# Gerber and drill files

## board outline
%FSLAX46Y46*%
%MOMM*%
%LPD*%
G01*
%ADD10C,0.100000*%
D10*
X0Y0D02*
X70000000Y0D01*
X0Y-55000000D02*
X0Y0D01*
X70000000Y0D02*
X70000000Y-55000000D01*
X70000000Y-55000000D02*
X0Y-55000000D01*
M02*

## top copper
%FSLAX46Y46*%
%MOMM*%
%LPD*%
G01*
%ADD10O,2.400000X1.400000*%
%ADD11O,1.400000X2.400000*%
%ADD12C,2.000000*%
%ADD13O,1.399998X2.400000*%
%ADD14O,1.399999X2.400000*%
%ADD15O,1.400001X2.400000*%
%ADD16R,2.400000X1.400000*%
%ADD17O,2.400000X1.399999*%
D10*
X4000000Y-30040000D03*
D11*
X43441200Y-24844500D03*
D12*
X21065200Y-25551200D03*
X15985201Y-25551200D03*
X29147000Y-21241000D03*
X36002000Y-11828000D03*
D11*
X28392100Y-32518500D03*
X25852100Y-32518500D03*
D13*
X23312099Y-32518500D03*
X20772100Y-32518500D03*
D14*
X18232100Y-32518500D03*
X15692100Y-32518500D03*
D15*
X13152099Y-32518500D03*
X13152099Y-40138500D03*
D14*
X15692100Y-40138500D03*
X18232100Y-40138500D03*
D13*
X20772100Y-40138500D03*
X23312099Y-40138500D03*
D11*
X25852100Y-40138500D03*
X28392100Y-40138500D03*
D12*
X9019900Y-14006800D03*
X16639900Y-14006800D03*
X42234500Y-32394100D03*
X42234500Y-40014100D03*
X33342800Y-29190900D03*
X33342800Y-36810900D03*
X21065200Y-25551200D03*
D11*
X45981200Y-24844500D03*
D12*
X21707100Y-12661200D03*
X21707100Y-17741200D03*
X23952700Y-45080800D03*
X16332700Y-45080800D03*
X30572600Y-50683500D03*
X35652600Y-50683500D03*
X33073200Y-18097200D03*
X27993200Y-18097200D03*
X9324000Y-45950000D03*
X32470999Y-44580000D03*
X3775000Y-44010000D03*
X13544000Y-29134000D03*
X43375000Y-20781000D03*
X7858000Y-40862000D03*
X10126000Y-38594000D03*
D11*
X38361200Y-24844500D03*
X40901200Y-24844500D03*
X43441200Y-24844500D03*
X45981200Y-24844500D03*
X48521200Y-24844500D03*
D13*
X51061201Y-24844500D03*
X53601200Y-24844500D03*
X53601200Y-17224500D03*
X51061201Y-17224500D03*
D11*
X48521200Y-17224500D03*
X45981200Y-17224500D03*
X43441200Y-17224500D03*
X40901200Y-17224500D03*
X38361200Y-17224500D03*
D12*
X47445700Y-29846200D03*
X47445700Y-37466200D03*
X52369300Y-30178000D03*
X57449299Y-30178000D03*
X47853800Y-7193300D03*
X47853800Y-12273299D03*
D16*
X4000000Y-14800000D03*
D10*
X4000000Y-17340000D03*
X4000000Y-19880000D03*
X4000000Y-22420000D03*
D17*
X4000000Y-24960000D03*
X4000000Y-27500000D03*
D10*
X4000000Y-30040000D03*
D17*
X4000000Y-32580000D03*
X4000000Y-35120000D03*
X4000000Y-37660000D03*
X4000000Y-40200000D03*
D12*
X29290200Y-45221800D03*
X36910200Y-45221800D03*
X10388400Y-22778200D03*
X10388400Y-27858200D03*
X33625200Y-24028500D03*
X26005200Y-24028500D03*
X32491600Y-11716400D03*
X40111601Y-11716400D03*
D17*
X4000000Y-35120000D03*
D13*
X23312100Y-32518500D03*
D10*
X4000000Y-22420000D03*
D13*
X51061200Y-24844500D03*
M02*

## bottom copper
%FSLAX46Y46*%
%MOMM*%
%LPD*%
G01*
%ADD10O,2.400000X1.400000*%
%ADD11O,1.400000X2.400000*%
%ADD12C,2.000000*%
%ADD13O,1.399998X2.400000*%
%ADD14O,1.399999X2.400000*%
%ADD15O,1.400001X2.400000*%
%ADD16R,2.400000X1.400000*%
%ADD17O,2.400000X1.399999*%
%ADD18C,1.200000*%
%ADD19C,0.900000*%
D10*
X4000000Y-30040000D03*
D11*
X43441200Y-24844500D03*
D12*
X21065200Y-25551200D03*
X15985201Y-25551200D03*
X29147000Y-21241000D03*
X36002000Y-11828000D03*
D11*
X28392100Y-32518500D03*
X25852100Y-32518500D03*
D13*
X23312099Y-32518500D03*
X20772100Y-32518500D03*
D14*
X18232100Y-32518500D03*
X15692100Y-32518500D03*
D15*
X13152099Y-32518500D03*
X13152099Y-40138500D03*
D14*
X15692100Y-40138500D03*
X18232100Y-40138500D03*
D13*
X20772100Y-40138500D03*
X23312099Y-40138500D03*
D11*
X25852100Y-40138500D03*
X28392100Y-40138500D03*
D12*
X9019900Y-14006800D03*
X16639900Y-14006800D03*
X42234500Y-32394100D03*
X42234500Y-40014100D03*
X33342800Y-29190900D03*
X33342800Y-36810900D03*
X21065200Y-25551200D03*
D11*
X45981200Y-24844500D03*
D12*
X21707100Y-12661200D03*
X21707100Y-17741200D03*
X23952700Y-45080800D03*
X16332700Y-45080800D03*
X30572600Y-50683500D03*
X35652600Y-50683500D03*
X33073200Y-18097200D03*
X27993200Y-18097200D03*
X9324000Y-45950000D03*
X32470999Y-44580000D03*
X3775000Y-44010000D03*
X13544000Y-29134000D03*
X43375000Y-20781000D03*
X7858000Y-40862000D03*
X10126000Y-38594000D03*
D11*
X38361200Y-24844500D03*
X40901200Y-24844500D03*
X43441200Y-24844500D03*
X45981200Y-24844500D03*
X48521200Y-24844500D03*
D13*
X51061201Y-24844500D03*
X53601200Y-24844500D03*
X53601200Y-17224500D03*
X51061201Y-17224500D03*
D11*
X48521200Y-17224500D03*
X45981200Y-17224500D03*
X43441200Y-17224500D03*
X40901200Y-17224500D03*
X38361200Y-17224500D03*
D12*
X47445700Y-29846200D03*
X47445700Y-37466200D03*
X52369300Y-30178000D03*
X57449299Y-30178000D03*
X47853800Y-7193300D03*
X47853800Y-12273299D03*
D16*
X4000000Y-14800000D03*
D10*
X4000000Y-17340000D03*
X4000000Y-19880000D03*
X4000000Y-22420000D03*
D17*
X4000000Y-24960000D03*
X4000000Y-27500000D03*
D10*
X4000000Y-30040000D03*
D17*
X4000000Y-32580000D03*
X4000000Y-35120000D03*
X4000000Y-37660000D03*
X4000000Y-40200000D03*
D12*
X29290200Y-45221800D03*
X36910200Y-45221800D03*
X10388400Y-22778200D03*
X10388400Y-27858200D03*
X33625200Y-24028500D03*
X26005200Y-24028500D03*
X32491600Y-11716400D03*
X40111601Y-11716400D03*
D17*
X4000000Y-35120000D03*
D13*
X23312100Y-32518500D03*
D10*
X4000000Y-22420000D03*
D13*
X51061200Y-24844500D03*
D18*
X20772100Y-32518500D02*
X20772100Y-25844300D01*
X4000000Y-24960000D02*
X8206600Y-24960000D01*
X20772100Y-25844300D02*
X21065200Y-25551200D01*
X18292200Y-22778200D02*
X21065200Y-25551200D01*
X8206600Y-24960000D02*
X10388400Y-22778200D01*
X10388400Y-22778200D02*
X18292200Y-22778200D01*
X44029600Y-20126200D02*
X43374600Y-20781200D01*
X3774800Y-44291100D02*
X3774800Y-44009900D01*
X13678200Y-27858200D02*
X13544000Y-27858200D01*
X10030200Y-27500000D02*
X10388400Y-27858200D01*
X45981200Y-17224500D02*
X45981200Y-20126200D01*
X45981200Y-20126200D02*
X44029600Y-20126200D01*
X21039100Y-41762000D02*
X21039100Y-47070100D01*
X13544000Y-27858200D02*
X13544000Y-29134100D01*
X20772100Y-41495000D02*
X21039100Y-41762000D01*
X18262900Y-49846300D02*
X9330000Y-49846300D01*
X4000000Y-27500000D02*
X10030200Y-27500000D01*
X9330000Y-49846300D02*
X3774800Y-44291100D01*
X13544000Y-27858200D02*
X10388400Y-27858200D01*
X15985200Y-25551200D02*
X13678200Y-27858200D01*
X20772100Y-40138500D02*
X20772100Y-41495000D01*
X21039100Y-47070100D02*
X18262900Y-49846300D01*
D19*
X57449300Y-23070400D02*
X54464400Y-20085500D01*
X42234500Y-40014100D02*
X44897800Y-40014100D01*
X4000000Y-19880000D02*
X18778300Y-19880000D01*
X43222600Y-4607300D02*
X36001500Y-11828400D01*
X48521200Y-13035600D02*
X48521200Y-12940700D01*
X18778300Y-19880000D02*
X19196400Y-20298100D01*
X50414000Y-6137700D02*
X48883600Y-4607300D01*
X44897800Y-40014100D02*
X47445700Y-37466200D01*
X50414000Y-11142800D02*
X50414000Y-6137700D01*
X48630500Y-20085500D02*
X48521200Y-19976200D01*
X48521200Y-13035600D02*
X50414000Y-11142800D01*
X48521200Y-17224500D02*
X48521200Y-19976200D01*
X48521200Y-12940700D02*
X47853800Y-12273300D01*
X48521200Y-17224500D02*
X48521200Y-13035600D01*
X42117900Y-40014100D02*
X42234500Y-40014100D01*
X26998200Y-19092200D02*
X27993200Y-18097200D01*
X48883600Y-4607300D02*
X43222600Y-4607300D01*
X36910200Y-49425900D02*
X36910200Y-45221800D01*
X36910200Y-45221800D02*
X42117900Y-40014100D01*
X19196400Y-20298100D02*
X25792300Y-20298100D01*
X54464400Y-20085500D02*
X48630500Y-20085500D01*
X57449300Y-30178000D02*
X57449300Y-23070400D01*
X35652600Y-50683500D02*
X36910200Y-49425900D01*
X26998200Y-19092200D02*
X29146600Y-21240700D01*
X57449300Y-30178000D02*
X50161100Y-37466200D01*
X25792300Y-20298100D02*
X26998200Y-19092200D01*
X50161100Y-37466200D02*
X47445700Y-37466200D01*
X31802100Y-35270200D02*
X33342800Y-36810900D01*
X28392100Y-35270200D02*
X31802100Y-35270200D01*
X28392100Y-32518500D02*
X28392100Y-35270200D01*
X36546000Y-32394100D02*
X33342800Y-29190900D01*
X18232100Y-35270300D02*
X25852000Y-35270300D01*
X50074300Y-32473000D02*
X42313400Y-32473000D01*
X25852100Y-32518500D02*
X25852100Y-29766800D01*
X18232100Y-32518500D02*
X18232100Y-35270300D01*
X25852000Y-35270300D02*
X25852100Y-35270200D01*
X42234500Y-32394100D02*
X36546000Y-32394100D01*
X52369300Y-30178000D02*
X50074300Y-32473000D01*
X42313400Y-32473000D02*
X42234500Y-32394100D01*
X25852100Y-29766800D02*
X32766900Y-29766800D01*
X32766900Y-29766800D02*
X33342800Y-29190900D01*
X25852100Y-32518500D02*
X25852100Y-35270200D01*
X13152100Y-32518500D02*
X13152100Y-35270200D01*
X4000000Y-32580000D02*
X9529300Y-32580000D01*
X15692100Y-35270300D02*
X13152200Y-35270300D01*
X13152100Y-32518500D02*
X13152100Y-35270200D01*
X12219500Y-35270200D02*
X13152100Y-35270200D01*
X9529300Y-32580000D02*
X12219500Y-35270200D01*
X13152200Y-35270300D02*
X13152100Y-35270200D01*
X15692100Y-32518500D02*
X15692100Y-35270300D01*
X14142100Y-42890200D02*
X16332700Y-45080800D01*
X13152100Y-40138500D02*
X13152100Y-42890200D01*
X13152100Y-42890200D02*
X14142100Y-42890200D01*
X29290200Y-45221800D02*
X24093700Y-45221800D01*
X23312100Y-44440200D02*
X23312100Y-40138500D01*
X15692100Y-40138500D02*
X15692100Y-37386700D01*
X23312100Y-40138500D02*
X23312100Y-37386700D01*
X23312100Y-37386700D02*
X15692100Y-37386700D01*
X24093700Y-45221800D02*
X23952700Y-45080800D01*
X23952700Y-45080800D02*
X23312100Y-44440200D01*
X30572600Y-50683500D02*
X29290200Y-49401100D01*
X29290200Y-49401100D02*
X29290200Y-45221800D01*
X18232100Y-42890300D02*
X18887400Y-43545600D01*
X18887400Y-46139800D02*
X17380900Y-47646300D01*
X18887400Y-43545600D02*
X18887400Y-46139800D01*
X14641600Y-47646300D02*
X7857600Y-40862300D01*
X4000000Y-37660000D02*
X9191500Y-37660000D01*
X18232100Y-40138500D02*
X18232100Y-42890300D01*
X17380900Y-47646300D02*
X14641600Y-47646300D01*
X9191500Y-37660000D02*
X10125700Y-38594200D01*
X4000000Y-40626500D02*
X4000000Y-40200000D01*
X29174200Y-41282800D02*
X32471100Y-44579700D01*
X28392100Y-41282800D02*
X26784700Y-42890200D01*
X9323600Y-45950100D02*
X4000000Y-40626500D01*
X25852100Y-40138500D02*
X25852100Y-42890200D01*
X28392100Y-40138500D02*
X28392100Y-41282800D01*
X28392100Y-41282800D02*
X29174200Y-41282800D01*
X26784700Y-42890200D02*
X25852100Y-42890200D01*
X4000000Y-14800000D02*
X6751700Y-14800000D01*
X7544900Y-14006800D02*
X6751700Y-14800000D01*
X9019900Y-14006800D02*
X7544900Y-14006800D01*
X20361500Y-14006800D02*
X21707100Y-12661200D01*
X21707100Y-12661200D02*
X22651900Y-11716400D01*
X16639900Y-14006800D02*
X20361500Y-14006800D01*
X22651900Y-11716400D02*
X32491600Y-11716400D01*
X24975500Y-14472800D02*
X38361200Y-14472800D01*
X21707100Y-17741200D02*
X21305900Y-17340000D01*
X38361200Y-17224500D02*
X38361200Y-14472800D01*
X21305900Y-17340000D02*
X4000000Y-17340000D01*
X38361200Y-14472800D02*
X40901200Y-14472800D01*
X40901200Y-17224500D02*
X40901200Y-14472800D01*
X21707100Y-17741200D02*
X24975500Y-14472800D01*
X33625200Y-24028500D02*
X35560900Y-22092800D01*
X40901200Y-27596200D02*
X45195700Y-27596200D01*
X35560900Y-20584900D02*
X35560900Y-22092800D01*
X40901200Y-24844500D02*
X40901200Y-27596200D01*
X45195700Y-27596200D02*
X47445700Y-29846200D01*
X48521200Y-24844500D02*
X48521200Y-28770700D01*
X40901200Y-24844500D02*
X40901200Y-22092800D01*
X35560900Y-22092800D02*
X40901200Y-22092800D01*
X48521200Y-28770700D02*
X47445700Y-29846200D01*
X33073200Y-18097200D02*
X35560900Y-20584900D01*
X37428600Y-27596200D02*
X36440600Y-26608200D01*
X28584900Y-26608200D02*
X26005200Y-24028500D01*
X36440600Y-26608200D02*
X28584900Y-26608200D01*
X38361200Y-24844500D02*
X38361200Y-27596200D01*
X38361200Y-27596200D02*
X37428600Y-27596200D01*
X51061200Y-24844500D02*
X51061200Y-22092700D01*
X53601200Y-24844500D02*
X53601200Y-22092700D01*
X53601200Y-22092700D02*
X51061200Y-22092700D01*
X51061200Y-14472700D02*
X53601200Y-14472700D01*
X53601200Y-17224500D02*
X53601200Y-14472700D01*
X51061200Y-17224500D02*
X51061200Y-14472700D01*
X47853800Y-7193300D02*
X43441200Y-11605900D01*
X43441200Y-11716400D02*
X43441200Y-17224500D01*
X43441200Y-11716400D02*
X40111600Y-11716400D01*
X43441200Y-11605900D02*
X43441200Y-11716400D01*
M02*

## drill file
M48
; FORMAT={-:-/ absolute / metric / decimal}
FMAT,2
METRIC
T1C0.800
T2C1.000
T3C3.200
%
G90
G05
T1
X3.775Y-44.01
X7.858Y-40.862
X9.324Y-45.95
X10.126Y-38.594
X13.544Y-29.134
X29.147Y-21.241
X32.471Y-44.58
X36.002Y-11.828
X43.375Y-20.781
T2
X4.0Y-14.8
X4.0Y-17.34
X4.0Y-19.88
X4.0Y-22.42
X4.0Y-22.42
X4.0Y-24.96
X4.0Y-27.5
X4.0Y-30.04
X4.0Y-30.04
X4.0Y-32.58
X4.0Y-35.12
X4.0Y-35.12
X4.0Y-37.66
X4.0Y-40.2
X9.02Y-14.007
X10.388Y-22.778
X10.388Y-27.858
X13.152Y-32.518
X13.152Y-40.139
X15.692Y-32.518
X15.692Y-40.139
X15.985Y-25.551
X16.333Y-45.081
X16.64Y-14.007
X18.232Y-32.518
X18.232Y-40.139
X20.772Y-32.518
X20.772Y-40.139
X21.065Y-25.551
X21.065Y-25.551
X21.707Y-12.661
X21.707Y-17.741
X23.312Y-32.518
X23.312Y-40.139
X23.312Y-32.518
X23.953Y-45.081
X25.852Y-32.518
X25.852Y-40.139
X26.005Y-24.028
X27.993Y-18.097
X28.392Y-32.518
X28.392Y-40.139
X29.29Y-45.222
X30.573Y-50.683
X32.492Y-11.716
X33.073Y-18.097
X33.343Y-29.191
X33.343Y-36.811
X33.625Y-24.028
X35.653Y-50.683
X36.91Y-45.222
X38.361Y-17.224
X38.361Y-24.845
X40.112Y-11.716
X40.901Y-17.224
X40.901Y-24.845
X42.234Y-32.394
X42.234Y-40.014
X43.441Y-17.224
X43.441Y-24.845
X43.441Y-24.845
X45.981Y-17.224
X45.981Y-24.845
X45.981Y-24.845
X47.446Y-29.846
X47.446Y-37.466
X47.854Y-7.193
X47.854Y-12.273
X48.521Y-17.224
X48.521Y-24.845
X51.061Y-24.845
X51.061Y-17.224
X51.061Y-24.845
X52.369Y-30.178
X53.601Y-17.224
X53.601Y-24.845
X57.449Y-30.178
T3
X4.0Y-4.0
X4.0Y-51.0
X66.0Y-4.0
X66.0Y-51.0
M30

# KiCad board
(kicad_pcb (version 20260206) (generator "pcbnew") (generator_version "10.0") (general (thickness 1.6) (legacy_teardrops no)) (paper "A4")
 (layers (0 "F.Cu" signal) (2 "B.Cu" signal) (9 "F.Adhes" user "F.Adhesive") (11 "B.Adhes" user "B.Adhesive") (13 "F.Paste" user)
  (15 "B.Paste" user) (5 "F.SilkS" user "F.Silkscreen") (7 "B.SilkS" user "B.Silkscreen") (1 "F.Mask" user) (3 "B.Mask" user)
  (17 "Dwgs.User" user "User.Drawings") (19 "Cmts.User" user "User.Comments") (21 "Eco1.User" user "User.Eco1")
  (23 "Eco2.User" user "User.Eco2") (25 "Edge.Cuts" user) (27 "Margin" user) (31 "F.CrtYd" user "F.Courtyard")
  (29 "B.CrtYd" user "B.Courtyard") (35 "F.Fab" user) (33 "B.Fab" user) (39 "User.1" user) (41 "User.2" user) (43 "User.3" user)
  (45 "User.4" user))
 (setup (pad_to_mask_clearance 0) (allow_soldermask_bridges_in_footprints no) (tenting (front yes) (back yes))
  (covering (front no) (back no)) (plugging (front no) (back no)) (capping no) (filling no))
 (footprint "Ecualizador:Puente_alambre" (layer "F.Cu") (at 4 30.04)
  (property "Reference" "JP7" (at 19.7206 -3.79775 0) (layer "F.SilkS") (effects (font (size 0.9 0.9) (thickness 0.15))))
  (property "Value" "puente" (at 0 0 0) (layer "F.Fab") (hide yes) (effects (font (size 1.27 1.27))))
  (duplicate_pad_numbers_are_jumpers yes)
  (pad "1" thru_hole oval (at 0 0) (size 2.4 1.4) (drill 1) (layers "*.Cu" "*.Mask") (remove_unused_layers no) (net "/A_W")
   (thermal_bridge_angle 45))
  (pad "1" thru_hole oval (at 39.4412 -5.1955 90) (size 2.4 1.4) (drill 1) (layers "*.Cu" "*.Mask") (remove_unused_layers no) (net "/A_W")
   (thermal_bridge_angle 45)))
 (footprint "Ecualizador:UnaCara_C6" (layer "F.Cu") (at 21.0652 25.5512 180)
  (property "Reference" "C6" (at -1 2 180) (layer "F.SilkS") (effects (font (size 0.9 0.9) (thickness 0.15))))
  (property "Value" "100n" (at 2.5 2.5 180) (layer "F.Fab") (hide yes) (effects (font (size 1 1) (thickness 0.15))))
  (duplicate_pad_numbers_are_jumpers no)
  (pad "1" thru_hole circle (at 0 0 180) (size 2 2) (drill 1) (layers "*.Cu" "*.Mask") (remove_unused_layers no) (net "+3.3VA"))
  (pad "2" thru_hole circle (at 5.079999 0 180) (size 2 2) (drill 1) (layers "*.Cu" "*.Mask") (remove_unused_layers no) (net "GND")))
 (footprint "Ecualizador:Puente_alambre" (layer "F.Cu") (at 29.147 21.241)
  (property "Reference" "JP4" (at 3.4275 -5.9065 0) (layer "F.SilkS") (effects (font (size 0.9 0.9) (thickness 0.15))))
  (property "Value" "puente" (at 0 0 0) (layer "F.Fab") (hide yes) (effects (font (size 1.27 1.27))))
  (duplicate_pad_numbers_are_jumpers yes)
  (pad "1" thru_hole circle (at 0 0) (size 2 2) (drill 0.8) (layers "*.Cu" "*.Mask") (remove_unused_layers no) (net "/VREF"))
  (pad "1" thru_hole circle (at 6.855 -9.413) (size 2 2) (drill 0.8) (layers "*.Cu" "*.Mask") (remove_unused_layers no) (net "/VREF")))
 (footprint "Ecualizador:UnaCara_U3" (layer "F.Cu") (at 28.3921 32.5185 -90)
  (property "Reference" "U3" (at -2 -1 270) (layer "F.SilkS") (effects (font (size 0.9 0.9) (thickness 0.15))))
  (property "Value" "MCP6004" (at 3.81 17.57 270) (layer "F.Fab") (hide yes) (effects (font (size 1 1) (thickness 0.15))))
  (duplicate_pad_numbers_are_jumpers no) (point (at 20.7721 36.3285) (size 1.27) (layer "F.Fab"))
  (pad "1" thru_hole oval (at 0 0 270) (size 2.4 1.4) (drill 1) (layers "*.Cu" "*.Mask") (remove_unused_layers no) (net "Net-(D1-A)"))
  (pad "2" thru_hole oval (at 0 2.54 270) (size 2.4 1.4) (drill 1) (layers "*.Cu" "*.Mask") (remove_unused_layers no) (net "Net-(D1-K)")
   (thermal_bridge_angle 45))
  (pad "3" thru_hole oval (at 0 5.080001 270) (size 2.4 1.399998) (drill 1) (layers "*.Cu" "*.Mask") (remove_unused_layers no) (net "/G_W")
   (thermal_bridge_angle 45))
  (pad "4" thru_hole oval (at 0 7.62 270) (size 2.4 1.399998) (drill 1) (layers "*.Cu" "*.Mask") (remove_unused_layers no) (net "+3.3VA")
   (thermal_bridge_angle 45))
  (pad "5" thru_hole oval (at 0 10.16 270) (size 2.4 1.399999) (drill 1) (layers "*.Cu" "*.Mask") (remove_unused_layers no)
   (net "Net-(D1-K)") (thermal_bridge_angle 45))
  (pad "6" thru_hole oval (at 0 12.7 270) (size 2.4 1.399999) (drill 1) (layers "*.Cu" "*.Mask") (remove_unused_layers no) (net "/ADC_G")
   (thermal_bridge_angle 45))
  (pad "7" thru_hole oval (at 0 15.240001 270) (size 2.4 1.400001) (drill 1) (layers "*.Cu" "*.Mask") (remove_unused_layers no)
   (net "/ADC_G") (thermal_bridge_angle 45))
  (pad "8" thru_hole oval (at 7.62 15.240001 270) (size 2.4 1.400001) (drill 1) (layers "*.Cu" "*.Mask") (remove_unused_layers no)
   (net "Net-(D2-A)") (thermal_bridge_angle 45))
  (pad "9" thru_hole oval (at 7.62 12.7 270) (size 2.4 1.399999) (drill 1) (layers "*.Cu" "*.Mask") (remove_unused_layers no)
   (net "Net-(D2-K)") (thermal_bridge_angle 45))
  (pad "10" thru_hole oval (at 7.62 10.16 270) (size 2.4 1.399999) (drill 1) (layers "*.Cu" "*.Mask") (remove_unused_layers no) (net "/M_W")
   (thermal_bridge_angle 45))
  (pad "11" thru_hole oval (at 7.62 7.62 270) (size 2.4 1.399998) (drill 1) (layers "*.Cu" "*.Mask") (remove_unused_layers no) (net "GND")
   (thermal_bridge_angle 45))
  (pad "12" thru_hole oval (at 7.62 5.080001 270) (size 2.4 1.399998) (drill 1) (layers "*.Cu" "*.Mask") (remove_unused_layers no)
   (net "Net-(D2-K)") (thermal_bridge_angle 45))
  (pad "13" thru_hole oval (at 7.62 2.54 270) (size 2.4 1.4) (drill 1) (layers "*.Cu" "*.Mask") (remove_unused_layers no) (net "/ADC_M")
   (thermal_bridge_angle 45))
  (pad "14" thru_hole oval (at 7.62 0 270) (size 2.4 1.4) (drill 1) (layers "*.Cu" "*.Mask") (remove_unused_layers no) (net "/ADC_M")
   (thermal_bridge_angle 45)))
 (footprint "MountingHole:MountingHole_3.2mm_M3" (layer "F.Cu") (at 4 4)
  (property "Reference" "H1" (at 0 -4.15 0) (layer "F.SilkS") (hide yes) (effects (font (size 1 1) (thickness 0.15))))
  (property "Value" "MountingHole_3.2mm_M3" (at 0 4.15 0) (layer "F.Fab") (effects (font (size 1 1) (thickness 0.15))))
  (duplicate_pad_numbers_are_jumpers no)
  (pad "" np_thru_hole circle (at 0 0) (size 3.2 3.2) (drill 3.2) (layers "*.Cu" "*.Mask")))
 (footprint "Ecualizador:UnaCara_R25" (layer "F.Cu") (at 9.0199 14.0068)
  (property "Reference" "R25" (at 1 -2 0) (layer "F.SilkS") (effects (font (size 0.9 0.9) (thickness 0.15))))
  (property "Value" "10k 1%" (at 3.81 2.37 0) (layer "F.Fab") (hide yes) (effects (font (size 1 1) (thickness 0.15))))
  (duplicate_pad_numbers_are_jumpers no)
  (pad "1" thru_hole circle (at 0 0) (size 2 2) (drill 1) (layers "*.Cu" "*.Mask") (remove_unused_layers no) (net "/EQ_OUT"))
  (pad "2" thru_hole circle (at 7.62 0) (size 2 2) (drill 1) (layers "*.Cu" "*.Mask") (remove_unused_layers no) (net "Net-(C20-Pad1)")))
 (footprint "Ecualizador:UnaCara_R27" (layer "F.Cu") (at 42.2345 32.3941 -90)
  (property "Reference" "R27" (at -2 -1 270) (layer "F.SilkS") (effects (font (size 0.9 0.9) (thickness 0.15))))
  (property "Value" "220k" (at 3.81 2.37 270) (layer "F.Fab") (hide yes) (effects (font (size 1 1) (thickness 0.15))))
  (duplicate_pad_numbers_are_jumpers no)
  (pad "1" thru_hole circle (at 0 0 270) (size 2 2) (drill 1) (layers "*.Cu" "*.Mask") (remove_unused_layers no) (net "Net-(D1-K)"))
  (pad "2" thru_hole circle (at 7.62 0 270) (size 2 2) (drill 1) (layers "*.Cu" "*.Mask") (remove_unused_layers no) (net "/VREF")))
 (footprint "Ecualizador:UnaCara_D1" (layer "F.Cu") (at 33.3428 29.1909 -90)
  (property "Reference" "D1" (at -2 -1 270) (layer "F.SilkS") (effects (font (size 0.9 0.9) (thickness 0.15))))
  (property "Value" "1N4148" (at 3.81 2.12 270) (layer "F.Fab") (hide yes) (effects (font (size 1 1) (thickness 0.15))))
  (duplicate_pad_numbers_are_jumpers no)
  (pad "1" thru_hole circle (at 0 0 270) (size 2 2) (drill 1) (layers "*.Cu" "*.Mask") (remove_unused_layers no) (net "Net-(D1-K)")
   (thermal_bridge_angle 90))
  (pad "2" thru_hole circle (at 7.62 0 270) (size 2 2) (drill 1) (layers "*.Cu" "*.Mask") (remove_unused_layers no) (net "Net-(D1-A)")))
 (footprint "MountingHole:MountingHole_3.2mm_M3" (layer "F.Cu") (at 4 51)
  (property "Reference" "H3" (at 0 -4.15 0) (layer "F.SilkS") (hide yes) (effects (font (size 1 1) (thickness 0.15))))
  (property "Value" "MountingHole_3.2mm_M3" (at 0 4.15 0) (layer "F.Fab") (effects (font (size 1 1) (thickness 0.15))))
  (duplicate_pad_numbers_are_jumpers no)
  (pad "" np_thru_hole circle (at 0 0) (size 3.2 3.2) (drill 3.2) (layers "*.Cu" "*.Mask")))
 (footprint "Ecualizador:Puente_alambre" (layer "F.Cu") (at 45.9812 24.8445)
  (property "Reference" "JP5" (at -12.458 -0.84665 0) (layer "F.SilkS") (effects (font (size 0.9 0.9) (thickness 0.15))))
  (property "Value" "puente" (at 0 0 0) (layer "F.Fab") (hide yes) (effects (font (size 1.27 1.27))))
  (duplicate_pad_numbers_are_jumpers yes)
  (pad "1" thru_hole circle (at -24.916 0.7067 180) (size 2 2) (drill 1) (layers "*.Cu" "*.Mask") (remove_unused_layers no) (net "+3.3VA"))
  (pad "1" thru_hole oval (at 0 0 90) (size 2.4 1.4) (drill 1) (layers "*.Cu" "*.Mask") (remove_unused_layers no) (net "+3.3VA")
   (thermal_bridge_angle 45)))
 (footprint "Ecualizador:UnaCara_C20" (layer "F.Cu") (at 21.7071 12.6612 -90)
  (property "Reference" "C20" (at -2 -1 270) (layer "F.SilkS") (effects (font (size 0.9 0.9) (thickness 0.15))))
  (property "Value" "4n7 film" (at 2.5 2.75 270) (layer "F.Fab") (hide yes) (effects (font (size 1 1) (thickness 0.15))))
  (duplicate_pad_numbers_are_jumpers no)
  (pad "1" thru_hole circle (at 0 0 270) (size 2 2) (drill 1) (layers "*.Cu" "*.Mask") (remove_unused_layers no) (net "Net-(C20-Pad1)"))
  (pad "2" thru_hole circle (at 5.08 0 270) (size 2 2) (drill 1) (layers "*.Cu" "*.Mask") (remove_unused_layers no) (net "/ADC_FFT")))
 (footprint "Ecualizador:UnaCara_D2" (layer "F.Cu") (at 23.9527 45.0808 180)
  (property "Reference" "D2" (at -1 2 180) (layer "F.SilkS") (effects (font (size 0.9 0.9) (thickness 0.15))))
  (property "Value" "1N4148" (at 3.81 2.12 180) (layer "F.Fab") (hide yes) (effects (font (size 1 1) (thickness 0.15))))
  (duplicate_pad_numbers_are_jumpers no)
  (pad "1" thru_hole circle (at 0 0 180) (size 2 2) (drill 1) (layers "*.Cu" "*.Mask") (remove_unused_layers no) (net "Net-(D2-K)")
   (thermal_bridge_angle 90))
  (pad "2" thru_hole circle (at 7.62 0 180) (size 2 2) (drill 1) (layers "*.Cu" "*.Mask") (remove_unused_layers no) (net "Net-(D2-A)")))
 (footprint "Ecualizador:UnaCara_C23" (layer "F.Cu") (at 30.5726 50.6835)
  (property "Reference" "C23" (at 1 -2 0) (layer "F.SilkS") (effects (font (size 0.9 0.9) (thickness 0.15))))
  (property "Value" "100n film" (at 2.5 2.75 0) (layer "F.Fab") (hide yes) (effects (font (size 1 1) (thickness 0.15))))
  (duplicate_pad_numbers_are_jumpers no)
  (pad "1" thru_hole circle (at 0 0) (size 2 2) (drill 1) (layers "*.Cu" "*.Mask") (remove_unused_layers no) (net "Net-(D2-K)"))
  (pad "2" thru_hole circle (at 5.08 0) (size 2 2) (drill 1) (layers "*.Cu" "*.Mask") (remove_unused_layers no) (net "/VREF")))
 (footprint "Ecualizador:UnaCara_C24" (layer "F.Cu") (at 33.0732 18.0972 180)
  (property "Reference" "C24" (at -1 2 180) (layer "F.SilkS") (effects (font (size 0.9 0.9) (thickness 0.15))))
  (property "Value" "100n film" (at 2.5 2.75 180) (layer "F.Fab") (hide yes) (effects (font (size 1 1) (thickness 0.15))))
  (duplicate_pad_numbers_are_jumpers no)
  (pad "1" thru_hole circle (at 0 0 180) (size 2 2) (drill 1) (layers "*.Cu" "*.Mask") (remove_unused_layers no) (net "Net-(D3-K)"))
  (pad "2" thru_hole circle (at 5.08 0 180) (size 2 2) (drill 1) (layers "*.Cu" "*.Mask") (remove_unused_layers no) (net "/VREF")))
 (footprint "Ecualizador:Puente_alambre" (layer "F.Cu") (at 9.324 45.95)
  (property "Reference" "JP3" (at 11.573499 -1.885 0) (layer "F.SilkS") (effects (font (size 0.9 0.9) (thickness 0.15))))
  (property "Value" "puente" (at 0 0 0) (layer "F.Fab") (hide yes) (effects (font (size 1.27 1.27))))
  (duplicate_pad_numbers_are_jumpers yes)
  (pad "1" thru_hole circle (at 0 0) (size 2 2) (drill 0.8) (layers "*.Cu" "*.Mask") (remove_unused_layers no) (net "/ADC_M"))
  (pad "1" thru_hole circle (at 23.146999 -1.37) (size 2 2) (drill 0.8) (layers "*.Cu" "*.Mask") (remove_unused_layers no) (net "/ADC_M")))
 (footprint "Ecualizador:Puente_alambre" (layer "F.Cu") (at 3.775 44.01)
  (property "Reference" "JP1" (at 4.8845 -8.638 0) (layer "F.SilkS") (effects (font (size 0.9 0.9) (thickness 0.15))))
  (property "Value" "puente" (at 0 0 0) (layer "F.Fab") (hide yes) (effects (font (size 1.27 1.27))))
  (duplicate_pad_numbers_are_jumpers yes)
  (pad "1" thru_hole circle (at 0 0) (size 2 2) (drill 0.8) (layers "*.Cu" "*.Mask") (remove_unused_layers no) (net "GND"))
  (pad "1" thru_hole circle (at 9.769 -14.876) (size 2 2) (drill 0.8) (layers "*.Cu" "*.Mask") (remove_unused_layers no) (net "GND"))
  (pad "1" thru_hole circle (at 39.6 -23.229) (size 2 2) (drill 0.8) (layers "*.Cu" "*.Mask") (remove_unused_layers no) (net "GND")))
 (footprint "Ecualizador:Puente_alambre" (layer "F.Cu") (at 7.858 40.862)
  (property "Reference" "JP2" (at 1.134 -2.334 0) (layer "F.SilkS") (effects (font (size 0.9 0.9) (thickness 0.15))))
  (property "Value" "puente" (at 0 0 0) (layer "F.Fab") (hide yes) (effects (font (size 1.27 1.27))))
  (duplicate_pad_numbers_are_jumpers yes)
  (pad "1" thru_hole circle (at 0 0) (size 2 2) (drill 0.8) (layers "*.Cu" "*.Mask") (remove_unused_layers no) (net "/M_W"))
  (pad "1" thru_hole circle (at 2.268 -2.268) (size 2 2) (drill 0.8) (layers "*.Cu" "*.Mask") (remove_unused_layers no) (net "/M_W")))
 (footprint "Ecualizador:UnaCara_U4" (layer "F.Cu") (at 38.3612 24.8445 90)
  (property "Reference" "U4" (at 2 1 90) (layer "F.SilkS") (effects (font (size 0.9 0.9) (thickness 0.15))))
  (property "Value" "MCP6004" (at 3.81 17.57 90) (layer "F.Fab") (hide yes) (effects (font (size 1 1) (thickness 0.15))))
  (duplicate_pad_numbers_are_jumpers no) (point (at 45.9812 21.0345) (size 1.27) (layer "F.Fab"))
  (pad "1" thru_hole oval (at 0 0 90) (size 2.4 1.4) (drill 1) (layers "*.Cu" "*.Mask") (remove_unused_layers no) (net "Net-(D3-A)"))
  (pad "2" thru_hole oval (at 0 2.54 90) (size 2.4 1.4) (drill 1) (layers "*.Cu" "*.Mask") (remove_unused_layers no) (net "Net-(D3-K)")
   (thermal_bridge_angle 45))
  (pad "3" thru_hole oval (at 0 5.08 90) (size 2.4 1.4) (drill 1) (layers "*.Cu" "*.Mask") (remove_unused_layers no) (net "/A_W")
   (thermal_bridge_angle 45))
  (pad "4" thru_hole oval (at 0 7.62 90) (size 2.4 1.4) (drill 1) (layers "*.Cu" "*.Mask") (remove_unused_layers no) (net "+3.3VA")
   (thermal_bridge_angle 45))
  (pad "5" thru_hole oval (at 0 10.16 90) (size 2.4 1.4) (drill 1) (layers "*.Cu" "*.Mask") (remove_unused_layers no) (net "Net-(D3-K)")
   (thermal_bridge_angle 45))
  (pad "6" thru_hole oval (at 0 12.700001 90) (size 2.4 1.399998) (drill 1) (layers "*.Cu" "*.Mask") (remove_unused_layers no)
   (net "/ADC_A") (thermal_bridge_angle 45))
  (pad "7" thru_hole oval (at 0 15.24 90) (size 2.4 1.399998) (drill 1) (layers "*.Cu" "*.Mask") (remove_unused_layers no) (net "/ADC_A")
   (thermal_bridge_angle 45))
  (pad "8" thru_hole oval (at 7.62 15.24 90) (size 2.4 1.399998) (drill 1) (layers "*.Cu" "*.Mask") (remove_unused_layers no)
   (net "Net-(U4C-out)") (thermal_bridge_angle 45))
  (pad "9" thru_hole oval (at 7.62 12.700001 90) (size 2.4 1.399998) (drill 1) (layers "*.Cu" "*.Mask") (remove_unused_layers no)
   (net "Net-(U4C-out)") (thermal_bridge_angle 45))
  (pad "10" thru_hole oval (at 7.62 10.16 90) (size 2.4 1.4) (drill 1) (layers "*.Cu" "*.Mask") (remove_unused_layers no) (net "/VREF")
   (thermal_bridge_angle 45))
  (pad "11" thru_hole oval (at 7.62 7.62 90) (size 2.4 1.4) (drill 1) (layers "*.Cu" "*.Mask") (remove_unused_layers no) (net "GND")
   (thermal_bridge_angle 45))
  (pad "12" thru_hole oval (at 7.62 5.08 90) (size 2.4 1.4) (drill 1) (layers "*.Cu" "*.Mask") (remove_unused_layers no) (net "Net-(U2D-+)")
   (thermal_bridge_angle 45))
  (pad "13" thru_hole oval (at 7.62 2.54 90) (size 2.4 1.4) (drill 1) (layers "*.Cu" "*.Mask") (remove_unused_layers no) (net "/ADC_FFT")
   (thermal_bridge_angle 45))
  (pad "14" thru_hole oval (at 7.62 0 90) (size 2.4 1.4) (drill 1) (layers "*.Cu" "*.Mask") (remove_unused_layers no) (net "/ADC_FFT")
   (thermal_bridge_angle 45)))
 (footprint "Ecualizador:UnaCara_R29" (layer "F.Cu") (at 47.4457 29.8462 -90)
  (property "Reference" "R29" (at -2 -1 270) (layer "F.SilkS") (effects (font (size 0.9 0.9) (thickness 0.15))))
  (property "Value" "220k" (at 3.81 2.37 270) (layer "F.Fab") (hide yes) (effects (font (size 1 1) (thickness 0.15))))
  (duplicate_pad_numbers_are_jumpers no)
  (pad "1" thru_hole circle (at 0 0 270) (size 2 2) (drill 1) (layers "*.Cu" "*.Mask") (remove_unused_layers no) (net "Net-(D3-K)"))
  (pad "2" thru_hole circle (at 7.62 0 270) (size 2 2) (drill 1) (layers "*.Cu" "*.Mask") (remove_unused_layers no) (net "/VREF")))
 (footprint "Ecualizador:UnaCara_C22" (layer "F.Cu") (at 52.3693 30.178)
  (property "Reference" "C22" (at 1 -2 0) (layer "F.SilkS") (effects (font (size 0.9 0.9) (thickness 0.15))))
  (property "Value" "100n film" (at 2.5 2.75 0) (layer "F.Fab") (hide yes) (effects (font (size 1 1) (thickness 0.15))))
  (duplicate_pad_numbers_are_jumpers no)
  (pad "1" thru_hole circle (at 0 0) (size 2 2) (drill 1) (layers "*.Cu" "*.Mask") (remove_unused_layers no) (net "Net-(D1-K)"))
  (pad "2" thru_hole circle (at 5.079999 0) (size 2 2) (drill 1) (layers "*.Cu" "*.Mask") (remove_unused_layers no) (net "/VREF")))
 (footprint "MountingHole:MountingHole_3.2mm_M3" (layer "F.Cu") (at 66 51)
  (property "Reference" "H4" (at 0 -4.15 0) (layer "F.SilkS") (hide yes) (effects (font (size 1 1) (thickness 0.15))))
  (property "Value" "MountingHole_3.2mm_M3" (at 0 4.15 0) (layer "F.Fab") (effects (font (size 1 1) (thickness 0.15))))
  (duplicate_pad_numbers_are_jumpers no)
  (pad "" np_thru_hole circle (at 0 0) (size 3.2 3.2) (drill 3.2) (layers "*.Cu" "*.Mask")))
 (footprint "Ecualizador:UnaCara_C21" (layer "F.Cu") (at 47.8538 7.1933 -90)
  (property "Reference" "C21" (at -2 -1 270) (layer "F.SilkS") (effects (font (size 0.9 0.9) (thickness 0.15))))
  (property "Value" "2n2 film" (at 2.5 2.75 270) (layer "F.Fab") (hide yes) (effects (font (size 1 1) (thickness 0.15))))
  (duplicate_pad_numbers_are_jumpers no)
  (pad "1" thru_hole circle (at 0 0 270) (size 2 2) (drill 1) (layers "*.Cu" "*.Mask") (remove_unused_layers no) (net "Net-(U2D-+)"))
  (pad "2" thru_hole circle (at 5.079999 0 270) (size 2 2) (drill 1) (layers "*.Cu" "*.Mask") (remove_unused_layers no) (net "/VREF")))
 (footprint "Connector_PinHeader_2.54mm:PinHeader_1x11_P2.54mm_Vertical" (layer "F.Cu") (at 4 14.8)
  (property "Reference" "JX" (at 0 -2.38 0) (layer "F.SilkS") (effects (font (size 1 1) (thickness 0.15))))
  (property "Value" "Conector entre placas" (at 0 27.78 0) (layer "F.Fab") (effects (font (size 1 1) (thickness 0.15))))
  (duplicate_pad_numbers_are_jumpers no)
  (pad "1" thru_hole rect (at 0 0) (size 2.4 1.4) (drill 1) (layers "*.Cu" "*.Mask") (remove_unused_layers no) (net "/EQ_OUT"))
  (pad "2" thru_hole oval (at 0 2.54) (size 2.4 1.4) (drill 1) (layers "*.Cu" "*.Mask") (remove_unused_layers no) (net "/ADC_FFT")
   (thermal_bridge_angle 45))
  (pad "3" thru_hole oval (at 0 5.08) (size 2.4 1.4) (drill 1) (layers "*.Cu" "*.Mask") (remove_unused_layers no) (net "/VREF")
   (thermal_bridge_angle 45))
  (pad "4" thru_hole oval (at 0 7.62) (size 2.4 1.4) (drill 1) (layers "*.Cu" "*.Mask") (remove_unused_layers no) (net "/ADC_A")
   (thermal_bridge_angle 45))
  (pad "5" thru_hole oval (at 0 10.16) (size 2.4 1.399999) (drill 1) (layers "*.Cu" "*.Mask") (remove_unused_layers no) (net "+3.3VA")
   (thermal_bridge_angle 45))
  (pad "6" thru_hole oval (at 0 12.7) (size 2.4 1.399999) (drill 1) (layers "*.Cu" "*.Mask") (remove_unused_layers no) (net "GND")
   (thermal_bridge_angle 45))
  (pad "7" thru_hole oval (at 0 15.24) (size 2.4 1.4) (drill 1) (layers "*.Cu" "*.Mask") (remove_unused_layers no) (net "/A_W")
   (thermal_bridge_angle 45))
  (pad "8" thru_hole oval (at 0 17.78) (size 2.4 1.399999) (drill 1) (layers "*.Cu" "*.Mask") (remove_unused_layers no) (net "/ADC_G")
   (thermal_bridge_angle 45))
  (pad "9" thru_hole oval (at 0 20.32) (size 2.4 1.399999) (drill 1) (layers "*.Cu" "*.Mask") (remove_unused_layers no) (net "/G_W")
   (thermal_bridge_angle 45))
  (pad "10" thru_hole oval (at 0 22.86) (size 2.4 1.399999) (drill 1) (layers "*.Cu" "*.Mask") (remove_unused_layers no) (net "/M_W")
   (thermal_bridge_angle 45))
  (pad "11" thru_hole oval (at 0 25.4) (size 2.4 1.399999) (drill 1) (layers "*.Cu" "*.Mask") (remove_unused_layers no) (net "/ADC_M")
   (thermal_bridge_angle 45)))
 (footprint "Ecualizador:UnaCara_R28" (layer "F.Cu") (at 29.2902 45.2218)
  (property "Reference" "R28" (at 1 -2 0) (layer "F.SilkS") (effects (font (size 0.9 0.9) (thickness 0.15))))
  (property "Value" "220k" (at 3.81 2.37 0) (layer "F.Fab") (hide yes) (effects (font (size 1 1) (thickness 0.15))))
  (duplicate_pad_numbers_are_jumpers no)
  (pad "1" thru_hole circle (at 0 0) (size 2 2) (drill 1) (layers "*.Cu" "*.Mask") (remove_unused_layers no) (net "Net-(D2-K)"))
  (pad "2" thru_hole circle (at 7.62 0) (size 2 2) (drill 1) (layers "*.Cu" "*.Mask") (remove_unused_layers no) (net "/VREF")))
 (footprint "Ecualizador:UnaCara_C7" (layer "F.Cu") (at 10.3884 22.7782 -90)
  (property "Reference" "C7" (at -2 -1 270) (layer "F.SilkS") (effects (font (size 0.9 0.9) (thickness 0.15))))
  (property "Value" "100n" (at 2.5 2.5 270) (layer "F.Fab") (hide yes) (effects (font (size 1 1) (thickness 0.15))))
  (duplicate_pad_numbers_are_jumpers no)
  (pad "1" thru_hole circle (at 0 0 270) (size 2 2) (drill 1) (layers "*.Cu" "*.Mask") (remove_unused_layers no) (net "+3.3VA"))
  (pad "2" thru_hole circle (at 5.08 0 270) (size 2 2) (drill 1) (layers "*.Cu" "*.Mask") (remove_unused_layers no) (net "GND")))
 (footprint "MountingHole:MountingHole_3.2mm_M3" (layer "F.Cu") (at 66 4)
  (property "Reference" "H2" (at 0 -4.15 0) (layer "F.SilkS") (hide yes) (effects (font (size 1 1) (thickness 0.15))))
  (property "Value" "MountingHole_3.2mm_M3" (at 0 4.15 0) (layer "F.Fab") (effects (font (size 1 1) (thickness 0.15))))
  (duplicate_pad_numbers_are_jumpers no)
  (pad "" np_thru_hole circle (at 0 0) (size 3.2 3.2) (drill 3.2) (layers "*.Cu" "*.Mask")))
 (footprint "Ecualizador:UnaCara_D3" (layer "F.Cu") (at 33.6252 24.0285 180)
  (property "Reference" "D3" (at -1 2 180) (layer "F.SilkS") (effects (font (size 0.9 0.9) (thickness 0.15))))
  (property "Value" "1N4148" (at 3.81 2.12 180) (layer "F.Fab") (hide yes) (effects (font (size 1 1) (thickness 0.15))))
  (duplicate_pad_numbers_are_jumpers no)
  (pad "1" thru_hole circle (at 0 0 180) (size 2 2) (drill 1) (layers "*.Cu" "*.Mask") (remove_unused_layers no) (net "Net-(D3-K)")
   (thermal_bridge_angle 90))
  (pad "2" thru_hole circle (at 7.62 0 180) (size 2 2) (drill 1) (layers "*.Cu" "*.Mask") (remove_unused_layers no) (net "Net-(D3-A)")))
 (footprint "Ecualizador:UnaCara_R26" (layer "F.Cu") (at 32.4916 11.7164)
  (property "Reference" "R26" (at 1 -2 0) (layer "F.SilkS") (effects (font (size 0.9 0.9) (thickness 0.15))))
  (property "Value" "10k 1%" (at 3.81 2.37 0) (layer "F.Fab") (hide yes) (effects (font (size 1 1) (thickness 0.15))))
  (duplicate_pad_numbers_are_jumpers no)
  (pad "1" thru_hole circle (at 0 0) (size 2 2) (drill 1) (layers "*.Cu" "*.Mask") (remove_unused_layers no) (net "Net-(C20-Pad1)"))
  (pad "2" thru_hole circle (at 7.620001 0) (size 2 2) (drill 1) (layers "*.Cu" "*.Mask") (remove_unused_layers no) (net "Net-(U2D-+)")))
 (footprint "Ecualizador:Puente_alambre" (layer "F.Cu") (at 4 35.12)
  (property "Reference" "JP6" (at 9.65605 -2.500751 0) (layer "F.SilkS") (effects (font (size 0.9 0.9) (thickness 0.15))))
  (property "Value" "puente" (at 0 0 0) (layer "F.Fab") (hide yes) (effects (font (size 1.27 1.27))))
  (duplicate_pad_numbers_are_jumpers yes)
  (pad "1" thru_hole oval (at 0 0) (size 2.4 1.399999) (drill 1) (layers "*.Cu" "*.Mask") (remove_unused_layers no) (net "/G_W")
   (thermal_bridge_angle 45))
  (pad "1" thru_hole oval (at 19.3121 -2.6015 270) (size 2.4 1.399998) (drill 1) (layers "*.Cu" "*.Mask") (remove_unused_layers no)
   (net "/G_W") (thermal_bridge_angle 45)))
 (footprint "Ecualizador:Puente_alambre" (layer "F.Cu") (at 51.0612 24.8445)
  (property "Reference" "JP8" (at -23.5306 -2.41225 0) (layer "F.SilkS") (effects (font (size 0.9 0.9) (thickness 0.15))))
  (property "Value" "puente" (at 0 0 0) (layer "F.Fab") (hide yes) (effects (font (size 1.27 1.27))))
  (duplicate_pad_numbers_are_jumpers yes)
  (pad "1" thru_hole oval (at -47.0612 -2.4245) (size 2.4 1.4) (drill 1) (layers "*.Cu" "*.Mask") (remove_unused_layers no) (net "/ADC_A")
   (thermal_bridge_angle 45))
  (pad "1" thru_hole oval (at 0 0 90) (size 2.4 1.399998) (drill 1) (layers "*.Cu" "*.Mask") (remove_unused_layers no) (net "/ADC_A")
   (thermal_bridge_angle 45)))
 (gr_line (start 0 0) (end 70 0) (stroke (width 0.1) (type default)) (layer "Edge.Cuts"))
 (gr_line (start 0 55) (end 0 0) (stroke (width 0.1) (type default)) (layer "Edge.Cuts"))
 (gr_line (start 70 0) (end 70 55) (stroke (width 0.1) (type default)) (layer "Edge.Cuts"))
 (gr_line (start 70 55) (end 0 55) (stroke (width 0.1) (type default)) (layer "Edge.Cuts"))
 (segment (start 20.7721 32.5185) (end 20.7721 25.8443) (width 1.2) (layer "B.Cu") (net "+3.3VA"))
 (segment (start 4 24.96) (end 8.2066 24.96) (width 1.2) (layer "B.Cu") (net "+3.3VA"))
 (segment (start 20.7721 25.8443) (end 21.0652 25.5512) (width 1.2) (layer "B.Cu") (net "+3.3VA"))
 (segment (start 18.2922 22.7782) (end 21.0652 25.5512) (width 1.2) (layer "B.Cu") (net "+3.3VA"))
 (segment (start 8.2066 24.96) (end 10.3884 22.7782) (width 1.2) (layer "B.Cu") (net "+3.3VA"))
 (segment (start 10.3884 22.7782) (end 18.2922 22.7782) (width 1.2) (layer "B.Cu") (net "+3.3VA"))
 (segment (start 44.0296 20.1262) (end 43.3746 20.7812) (width 1.2) (layer "B.Cu") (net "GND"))
 (segment (start 3.7748 44.2911) (end 3.7748 44.0099) (width 1.2) (layer "B.Cu") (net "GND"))
 (segment (start 13.6782 27.8582) (end 13.544 27.8582) (width 1.2) (layer "B.Cu") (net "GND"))
 (segment (start 10.0302 27.5) (end 10.3884 27.8582) (width 1.2) (layer "B.Cu") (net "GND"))
 (segment (start 45.9812 17.2245) (end 45.9812 20.1262) (width 1.2) (layer "B.Cu") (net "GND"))
 (segment (start 45.9812 20.1262) (end 44.0296 20.1262) (width 1.2) (layer "B.Cu") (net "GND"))
 (segment (start 21.0391 41.762) (end 21.0391 47.0701) (width 1.2) (layer "B.Cu") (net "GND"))
 (segment (start 13.544 27.8582) (end 13.544 29.1341) (width 1.2) (layer "B.Cu") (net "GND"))
 (segment (start 20.7721 41.495) (end 21.0391 41.762) (width 1.2) (layer "B.Cu") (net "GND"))
 (segment (start 18.2629 49.8463) (end 9.33 49.8463) (width 1.2) (layer "B.Cu") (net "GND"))
 (segment (start 4 27.5) (end 10.0302 27.5) (width 1.2) (layer "B.Cu") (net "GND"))
 (segment (start 9.33 49.8463) (end 3.7748 44.2911) (width 1.2) (layer "B.Cu") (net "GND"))
 (segment (start 13.544 27.8582) (end 10.3884 27.8582) (width 1.2) (layer "B.Cu") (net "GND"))
 (segment (start 15.9852 25.5512) (end 13.6782 27.8582) (width 1.2) (layer "B.Cu") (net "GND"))
 (segment (start 20.7721 40.1385) (end 20.7721 41.495) (width 1.2) (layer "B.Cu") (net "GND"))
 (segment (start 21.0391 47.0701) (end 18.2629 49.8463) (width 1.2) (layer "B.Cu") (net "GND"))
 (segment (start 57.4493 23.0704) (end 54.4644 20.0855) (width 0.9) (layer "B.Cu") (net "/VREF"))
 (segment (start 42.2345 40.0141) (end 44.8978 40.0141) (width 0.9) (layer "B.Cu") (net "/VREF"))
 (segment (start 4 19.88) (end 18.7783 19.88) (width 0.9) (layer "B.Cu") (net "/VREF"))
 (segment (start 43.2226 4.6073) (end 36.0015 11.8284) (width 0.9) (layer "B.Cu") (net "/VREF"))
 (segment (start 48.5212 13.0356) (end 48.5212 12.9407) (width 0.9) (layer "B.Cu") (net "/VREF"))
 (segment (start 18.7783 19.88) (end 19.1964 20.2981) (width 0.9) (layer "B.Cu") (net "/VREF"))
 (segment (start 50.414 6.1377) (end 48.8836 4.6073) (width 0.9) (layer "B.Cu") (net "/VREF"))
 (segment (start 44.8978 40.0141) (end 47.4457 37.4662) (width 0.9) (layer "B.Cu") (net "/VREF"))
 (segment (start 50.414 11.1428) (end 50.414 6.1377) (width 0.9) (layer "B.Cu") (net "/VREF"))
 (segment (start 48.6305 20.0855) (end 48.5212 19.9762) (width 0.9) (layer "B.Cu") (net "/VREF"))
 (segment (start 48.5212 13.0356) (end 50.414 11.1428) (width 0.9) (layer "B.Cu") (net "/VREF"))
 (segment (start 48.5212 17.2245) (end 48.5212 19.9762) (width 0.9) (layer "B.Cu") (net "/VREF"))
 (segment (start 48.5212 12.9407) (end 47.8538 12.2733) (width 0.9) (layer "B.Cu") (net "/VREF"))
 (segment (start 48.5212 17.2245) (end 48.5212 13.0356) (width 0.9) (layer "B.Cu") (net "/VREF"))
 (segment (start 42.1179 40.0141) (end 42.2345 40.0141) (width 0.9) (layer "B.Cu") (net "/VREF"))
 (segment (start 26.9982 19.0922) (end 27.9932 18.0972) (width 0.9) (layer "B.Cu") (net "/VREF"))
 (segment (start 48.8836 4.6073) (end 43.2226 4.6073) (width 0.9) (layer "B.Cu") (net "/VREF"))
 (segment (start 36.9102 49.4259) (end 36.9102 45.2218) (width 0.9) (layer "B.Cu") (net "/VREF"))
 (segment (start 36.9102 45.2218) (end 42.1179 40.0141) (width 0.9) (layer "B.Cu") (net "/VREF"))
 (segment (start 19.1964 20.2981) (end 25.7923 20.2981) (width 0.9) (layer "B.Cu") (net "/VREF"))
 (segment (start 54.4644 20.0855) (end 48.6305 20.0855) (width 0.9) (layer "B.Cu") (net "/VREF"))
 (segment (start 57.4493 30.178) (end 57.4493 23.0704) (width 0.9) (layer "B.Cu") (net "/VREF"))
 (segment (start 35.6526 50.6835) (end 36.9102 49.4259) (width 0.9) (layer "B.Cu") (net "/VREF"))
 (segment (start 26.9982 19.0922) (end 29.1466 21.2407) (width 0.9) (layer "B.Cu") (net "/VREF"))
 (segment (start 57.4493 30.178) (end 50.1611 37.4662) (width 0.9) (layer "B.Cu") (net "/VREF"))
 (segment (start 25.7923 20.2981) (end 26.9982 19.0922) (width 0.9) (layer "B.Cu") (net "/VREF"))
 (segment (start 50.1611 37.4662) (end 47.4457 37.4662) (width 0.9) (layer "B.Cu") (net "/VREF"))
 (segment (start 31.8021 35.2702) (end 33.3428 36.8109) (width 0.9) (layer "B.Cu") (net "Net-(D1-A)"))
 (segment (start 28.3921 35.2702) (end 31.8021 35.2702) (width 0.9) (layer "B.Cu") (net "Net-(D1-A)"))
 (segment (start 28.3921 32.5185) (end 28.3921 35.2702) (width 0.9) (layer "B.Cu") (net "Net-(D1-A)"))
 (segment (start 36.546 32.3941) (end 33.3428 29.1909) (width 0.9) (layer "B.Cu") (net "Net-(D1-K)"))
 (segment (start 18.2321 35.2703) (end 25.852 35.2703) (width 0.9) (layer "B.Cu") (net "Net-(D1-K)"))
 (segment (start 50.0743 32.473) (end 42.3134 32.473) (width 0.9) (layer "B.Cu") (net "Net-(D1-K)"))
 (segment (start 25.8521 32.5185) (end 25.8521 29.7668) (width 0.9) (layer "B.Cu") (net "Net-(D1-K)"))
 (segment (start 18.2321 32.5185) (end 18.2321 35.2703) (width 0.9) (layer "B.Cu") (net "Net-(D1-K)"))
 (segment (start 25.852 35.2703) (end 25.8521 35.2702) (width 0.9) (layer "B.Cu") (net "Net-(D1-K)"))
 (segment (start 42.2345 32.3941) (end 36.546 32.3941) (width 0.9) (layer "B.Cu") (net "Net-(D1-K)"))
 (segment (start 52.3693 30.178) (end 50.0743 32.473) (width 0.9) (layer "B.Cu") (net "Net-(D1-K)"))
 (segment (start 42.3134 32.473) (end 42.2345 32.3941) (width 0.9) (layer "B.Cu") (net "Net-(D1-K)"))
 (segment (start 25.8521 29.7668) (end 32.7669 29.7668) (width 0.9) (layer "B.Cu") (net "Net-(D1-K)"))
 (segment (start 32.7669 29.7668) (end 33.3428 29.1909) (width 0.9) (layer "B.Cu") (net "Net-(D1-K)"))
 (segment (start 25.8521 32.5185) (end 25.8521 35.2702) (width 0.9) (layer "B.Cu") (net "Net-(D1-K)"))
 (segment (start 13.1521 32.5185) (end 13.1521 35.2702) (width 0.9) (layer "B.Cu") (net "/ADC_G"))
 (segment (start 4 32.58) (end 9.5293 32.58) (width 0.9) (layer "B.Cu") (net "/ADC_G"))
 (segment (start 15.6921 35.2703) (end 13.1522 35.2703) (width 0.9) (layer "B.Cu") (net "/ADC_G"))
 (segment (start 13.1521 32.5185) (end 13.1521 35.2702) (width 0.9) (layer "B.Cu") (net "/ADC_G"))
 (segment (start 12.2195 35.2702) (end 13.1521 35.2702) (width 0.9) (layer "B.Cu") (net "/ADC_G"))
 (segment (start 9.5293 32.58) (end 12.2195 35.2702) (width 0.9) (layer "B.Cu") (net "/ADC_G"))
 (segment (start 13.1522 35.2703) (end 13.1521 35.2702) (width 0.9) (layer "B.Cu") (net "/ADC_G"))
 (segment (start 15.6921 32.5185) (end 15.6921 35.2703) (width 0.9) (layer "B.Cu") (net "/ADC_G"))
 (segment (start 14.1421 42.8902) (end 16.3327 45.0808) (width 0.9) (layer "B.Cu") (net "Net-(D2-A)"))
 (segment (start 13.1521 40.1385) (end 13.1521 42.8902) (width 0.9) (layer "B.Cu") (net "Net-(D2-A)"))
 (segment (start 13.1521 42.8902) (end 14.1421 42.8902) (width 0.9) (layer "B.Cu") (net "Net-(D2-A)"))
 (segment (start 29.2902 45.2218) (end 24.0937 45.2218) (width 0.9) (layer "B.Cu") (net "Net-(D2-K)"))
 (segment (start 23.3121 44.4402) (end 23.3121 40.1385) (width 0.9) (layer "B.Cu") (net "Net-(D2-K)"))
 (segment (start 15.6921 40.1385) (end 15.6921 37.3867) (width 0.9) (layer "B.Cu") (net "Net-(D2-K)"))
 (segment (start 23.3121 40.1385) (end 23.3121 37.3867) (width 0.9) (layer "B.Cu") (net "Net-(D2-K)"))
 (segment (start 23.3121 37.3867) (end 15.6921 37.3867) (width 0.9) (layer "B.Cu") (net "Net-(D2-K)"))
 (segment (start 24.0937 45.2218) (end 23.9527 45.0808) (width 0.9) (layer "B.Cu") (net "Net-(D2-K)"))
 (segment (start 23.9527 45.0808) (end 23.3121 44.4402) (width 0.9) (layer "B.Cu") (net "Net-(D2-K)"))
 (segment (start 30.5726 50.6835) (end 29.2902 49.4011) (width 0.9) (layer "B.Cu") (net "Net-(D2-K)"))
 (segment (start 29.2902 49.4011) (end 29.2902 45.2218) (width 0.9) (layer "B.Cu") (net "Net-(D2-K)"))
 (segment (start 18.2321 42.8903) (end 18.8874 43.5456) (width 0.9) (layer "B.Cu") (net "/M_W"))
 (segment (start 18.8874 46.1398) (end 17.3809 47.6463) (width 0.9) (layer "B.Cu") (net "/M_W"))
 (segment (start 18.8874 43.5456) (end 18.8874 46.1398) (width 0.9) (layer "B.Cu") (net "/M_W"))
 (segment (start 14.6416 47.6463) (end 7.8576 40.8623) (width 0.9) (layer "B.Cu") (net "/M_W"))
 (segment (start 4 37.66) (end 9.1915 37.66) (width 0.9) (layer "B.Cu") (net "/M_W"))
 (segment (start 18.2321 40.1385) (end 18.2321 42.8903) (width 0.9) (layer "B.Cu") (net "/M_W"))
 (segment (start 17.3809 47.6463) (end 14.6416 47.6463) (width 0.9) (layer "B.Cu") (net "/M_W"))
 (segment (start 9.1915 37.66) (end 10.1257 38.5942) (width 0.9) (layer "B.Cu") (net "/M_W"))
 (segment (start 4 40.6265) (end 4 40.2) (width 0.9) (layer "B.Cu") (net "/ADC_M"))
 (segment (start 29.1742 41.2828) (end 32.4711 44.5797) (width 0.9) (layer "B.Cu") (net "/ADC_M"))
 (segment (start 28.3921 41.2828) (end 26.7847 42.8902) (width 0.9) (layer "B.Cu") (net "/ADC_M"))
 (segment (start 9.3236 45.9501) (end 4 40.6265) (width 0.9) (layer "B.Cu") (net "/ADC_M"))
 (segment (start 25.8521 40.1385) (end 25.8521 42.8902) (width 0.9) (layer "B.Cu") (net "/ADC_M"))
 (segment (start 28.3921 40.1385) (end 28.3921 41.2828) (width 0.9) (layer "B.Cu") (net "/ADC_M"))
 (segment (start 28.3921 41.2828) (end 29.1742 41.2828) (width 0.9) (layer "B.Cu") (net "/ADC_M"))
 (segment (start 26.7847 42.8902) (end 25.8521 42.8902) (width 0.9) (layer "B.Cu") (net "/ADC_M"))
 (segment (start 4 14.8) (end 6.7517 14.8) (width 0.9) (layer "B.Cu") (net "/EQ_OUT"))
 (segment (start 7.5449 14.0068) (end 6.7517 14.8) (width 0.9) (layer "B.Cu") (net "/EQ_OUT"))
 (segment (start 9.0199 14.0068) (end 7.5449 14.0068) (width 0.9) (layer "B.Cu") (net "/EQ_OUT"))
 (segment (start 20.3615 14.0068) (end 21.7071 12.6612) (width 0.9) (layer "B.Cu") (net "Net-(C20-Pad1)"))
 (segment (start 21.7071 12.6612) (end 22.6519 11.7164) (width 0.9) (layer "B.Cu") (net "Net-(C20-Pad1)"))
 (segment (start 16.6399 14.0068) (end 20.3615 14.0068) (width 0.9) (layer "B.Cu") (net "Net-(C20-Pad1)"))
 (segment (start 22.6519 11.7164) (end 32.4916 11.7164) (width 0.9) (layer "B.Cu") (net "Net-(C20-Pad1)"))
 (segment (start 24.9755 14.4728) (end 38.3612 14.4728) (width 0.9) (layer "B.Cu") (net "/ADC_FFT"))
 (segment (start 21.7071 17.7412) (end 21.3059 17.34) (width 0.9) (layer "B.Cu") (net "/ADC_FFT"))
 (segment (start 38.3612 17.2245) (end 38.3612 14.4728) (width 0.9) (layer "B.Cu") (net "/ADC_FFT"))
 (segment (start 21.3059 17.34) (end 4 17.34) (width 0.9) (layer "B.Cu") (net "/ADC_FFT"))
 (segment (start 38.3612 14.4728) (end 40.9012 14.4728) (width 0.9) (layer "B.Cu") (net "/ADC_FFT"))
 (segment (start 40.9012 17.2245) (end 40.9012 14.4728) (width 0.9) (layer "B.Cu") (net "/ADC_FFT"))
 (segment (start 21.7071 17.7412) (end 24.9755 14.4728) (width 0.9) (layer "B.Cu") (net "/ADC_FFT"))
 (segment (start 33.6252 24.0285) (end 35.5609 22.0928) (width 0.9) (layer "B.Cu") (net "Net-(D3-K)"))
 (segment (start 40.9012 27.5962) (end 45.1957 27.5962) (width 0.9) (layer "B.Cu") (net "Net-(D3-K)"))
 (segment (start 35.5609 20.5849) (end 35.5609 22.0928) (width 0.9) (layer "B.Cu") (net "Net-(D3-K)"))
 (segment (start 40.9012 24.8445) (end 40.9012 27.5962) (width 0.9) (layer "B.Cu") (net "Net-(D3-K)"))
 (segment (start 45.1957 27.5962) (end 47.4457 29.8462) (width 0.9) (layer "B.Cu") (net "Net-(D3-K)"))
 (segment (start 48.5212 24.8445) (end 48.5212 28.7707) (width 0.9) (layer "B.Cu") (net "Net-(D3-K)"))
 (segment (start 40.9012 24.8445) (end 40.9012 22.0928) (width 0.9) (layer "B.Cu") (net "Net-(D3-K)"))
 (segment (start 35.5609 22.0928) (end 40.9012 22.0928) (width 0.9) (layer "B.Cu") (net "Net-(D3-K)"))
 (segment (start 48.5212 28.7707) (end 47.4457 29.8462) (width 0.9) (layer "B.Cu") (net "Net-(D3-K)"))
 (segment (start 33.0732 18.0972) (end 35.5609 20.5849) (width 0.9) (layer "B.Cu") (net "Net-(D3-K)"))
 (segment (start 37.4286 27.5962) (end 36.4406 26.6082) (width 0.9) (layer "B.Cu") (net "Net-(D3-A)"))
 (segment (start 28.5849 26.6082) (end 26.0052 24.0285) (width 0.9) (layer "B.Cu") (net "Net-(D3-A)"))
 (segment (start 36.4406 26.6082) (end 28.5849 26.6082) (width 0.9) (layer "B.Cu") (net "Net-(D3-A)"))
 (segment (start 38.3612 24.8445) (end 38.3612 27.5962) (width 0.9) (layer "B.Cu") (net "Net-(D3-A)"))
 (segment (start 38.3612 27.5962) (end 37.4286 27.5962) (width 0.9) (layer "B.Cu") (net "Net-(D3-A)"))
 (segment (start 51.0612 24.8445) (end 51.0612 22.0927) (width 0.9) (layer "B.Cu") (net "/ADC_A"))
 (segment (start 53.6012 24.8445) (end 53.6012 22.0927) (width 0.9) (layer "B.Cu") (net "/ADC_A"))
 (segment (start 53.6012 22.0927) (end 51.0612 22.0927) (width 0.9) (layer "B.Cu") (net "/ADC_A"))
 (segment (start 51.0612 14.4727) (end 53.6012 14.4727) (width 0.9) (layer "B.Cu") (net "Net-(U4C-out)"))
 (segment (start 53.6012 17.2245) (end 53.6012 14.4727) (width 0.9) (layer "B.Cu") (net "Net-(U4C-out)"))
 (segment (start 51.0612 17.2245) (end 51.0612 14.4727) (width 0.9) (layer "B.Cu") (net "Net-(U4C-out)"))
 (segment (start 47.8538 7.1933) (end 43.4412 11.6059) (width 0.9) (layer "B.Cu") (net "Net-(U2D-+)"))
 (segment (start 43.4412 11.7164) (end 43.4412 17.2245) (width 0.9) (layer "B.Cu") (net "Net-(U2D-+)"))
 (segment (start 43.4412 11.7164) (end 40.1116 11.7164) (width 0.9) (layer "B.Cu") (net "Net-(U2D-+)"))
 (segment (start 43.4412 11.6059) (end 43.4412 11.7164) (width 0.9) (layer "B.Cu") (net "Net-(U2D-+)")))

